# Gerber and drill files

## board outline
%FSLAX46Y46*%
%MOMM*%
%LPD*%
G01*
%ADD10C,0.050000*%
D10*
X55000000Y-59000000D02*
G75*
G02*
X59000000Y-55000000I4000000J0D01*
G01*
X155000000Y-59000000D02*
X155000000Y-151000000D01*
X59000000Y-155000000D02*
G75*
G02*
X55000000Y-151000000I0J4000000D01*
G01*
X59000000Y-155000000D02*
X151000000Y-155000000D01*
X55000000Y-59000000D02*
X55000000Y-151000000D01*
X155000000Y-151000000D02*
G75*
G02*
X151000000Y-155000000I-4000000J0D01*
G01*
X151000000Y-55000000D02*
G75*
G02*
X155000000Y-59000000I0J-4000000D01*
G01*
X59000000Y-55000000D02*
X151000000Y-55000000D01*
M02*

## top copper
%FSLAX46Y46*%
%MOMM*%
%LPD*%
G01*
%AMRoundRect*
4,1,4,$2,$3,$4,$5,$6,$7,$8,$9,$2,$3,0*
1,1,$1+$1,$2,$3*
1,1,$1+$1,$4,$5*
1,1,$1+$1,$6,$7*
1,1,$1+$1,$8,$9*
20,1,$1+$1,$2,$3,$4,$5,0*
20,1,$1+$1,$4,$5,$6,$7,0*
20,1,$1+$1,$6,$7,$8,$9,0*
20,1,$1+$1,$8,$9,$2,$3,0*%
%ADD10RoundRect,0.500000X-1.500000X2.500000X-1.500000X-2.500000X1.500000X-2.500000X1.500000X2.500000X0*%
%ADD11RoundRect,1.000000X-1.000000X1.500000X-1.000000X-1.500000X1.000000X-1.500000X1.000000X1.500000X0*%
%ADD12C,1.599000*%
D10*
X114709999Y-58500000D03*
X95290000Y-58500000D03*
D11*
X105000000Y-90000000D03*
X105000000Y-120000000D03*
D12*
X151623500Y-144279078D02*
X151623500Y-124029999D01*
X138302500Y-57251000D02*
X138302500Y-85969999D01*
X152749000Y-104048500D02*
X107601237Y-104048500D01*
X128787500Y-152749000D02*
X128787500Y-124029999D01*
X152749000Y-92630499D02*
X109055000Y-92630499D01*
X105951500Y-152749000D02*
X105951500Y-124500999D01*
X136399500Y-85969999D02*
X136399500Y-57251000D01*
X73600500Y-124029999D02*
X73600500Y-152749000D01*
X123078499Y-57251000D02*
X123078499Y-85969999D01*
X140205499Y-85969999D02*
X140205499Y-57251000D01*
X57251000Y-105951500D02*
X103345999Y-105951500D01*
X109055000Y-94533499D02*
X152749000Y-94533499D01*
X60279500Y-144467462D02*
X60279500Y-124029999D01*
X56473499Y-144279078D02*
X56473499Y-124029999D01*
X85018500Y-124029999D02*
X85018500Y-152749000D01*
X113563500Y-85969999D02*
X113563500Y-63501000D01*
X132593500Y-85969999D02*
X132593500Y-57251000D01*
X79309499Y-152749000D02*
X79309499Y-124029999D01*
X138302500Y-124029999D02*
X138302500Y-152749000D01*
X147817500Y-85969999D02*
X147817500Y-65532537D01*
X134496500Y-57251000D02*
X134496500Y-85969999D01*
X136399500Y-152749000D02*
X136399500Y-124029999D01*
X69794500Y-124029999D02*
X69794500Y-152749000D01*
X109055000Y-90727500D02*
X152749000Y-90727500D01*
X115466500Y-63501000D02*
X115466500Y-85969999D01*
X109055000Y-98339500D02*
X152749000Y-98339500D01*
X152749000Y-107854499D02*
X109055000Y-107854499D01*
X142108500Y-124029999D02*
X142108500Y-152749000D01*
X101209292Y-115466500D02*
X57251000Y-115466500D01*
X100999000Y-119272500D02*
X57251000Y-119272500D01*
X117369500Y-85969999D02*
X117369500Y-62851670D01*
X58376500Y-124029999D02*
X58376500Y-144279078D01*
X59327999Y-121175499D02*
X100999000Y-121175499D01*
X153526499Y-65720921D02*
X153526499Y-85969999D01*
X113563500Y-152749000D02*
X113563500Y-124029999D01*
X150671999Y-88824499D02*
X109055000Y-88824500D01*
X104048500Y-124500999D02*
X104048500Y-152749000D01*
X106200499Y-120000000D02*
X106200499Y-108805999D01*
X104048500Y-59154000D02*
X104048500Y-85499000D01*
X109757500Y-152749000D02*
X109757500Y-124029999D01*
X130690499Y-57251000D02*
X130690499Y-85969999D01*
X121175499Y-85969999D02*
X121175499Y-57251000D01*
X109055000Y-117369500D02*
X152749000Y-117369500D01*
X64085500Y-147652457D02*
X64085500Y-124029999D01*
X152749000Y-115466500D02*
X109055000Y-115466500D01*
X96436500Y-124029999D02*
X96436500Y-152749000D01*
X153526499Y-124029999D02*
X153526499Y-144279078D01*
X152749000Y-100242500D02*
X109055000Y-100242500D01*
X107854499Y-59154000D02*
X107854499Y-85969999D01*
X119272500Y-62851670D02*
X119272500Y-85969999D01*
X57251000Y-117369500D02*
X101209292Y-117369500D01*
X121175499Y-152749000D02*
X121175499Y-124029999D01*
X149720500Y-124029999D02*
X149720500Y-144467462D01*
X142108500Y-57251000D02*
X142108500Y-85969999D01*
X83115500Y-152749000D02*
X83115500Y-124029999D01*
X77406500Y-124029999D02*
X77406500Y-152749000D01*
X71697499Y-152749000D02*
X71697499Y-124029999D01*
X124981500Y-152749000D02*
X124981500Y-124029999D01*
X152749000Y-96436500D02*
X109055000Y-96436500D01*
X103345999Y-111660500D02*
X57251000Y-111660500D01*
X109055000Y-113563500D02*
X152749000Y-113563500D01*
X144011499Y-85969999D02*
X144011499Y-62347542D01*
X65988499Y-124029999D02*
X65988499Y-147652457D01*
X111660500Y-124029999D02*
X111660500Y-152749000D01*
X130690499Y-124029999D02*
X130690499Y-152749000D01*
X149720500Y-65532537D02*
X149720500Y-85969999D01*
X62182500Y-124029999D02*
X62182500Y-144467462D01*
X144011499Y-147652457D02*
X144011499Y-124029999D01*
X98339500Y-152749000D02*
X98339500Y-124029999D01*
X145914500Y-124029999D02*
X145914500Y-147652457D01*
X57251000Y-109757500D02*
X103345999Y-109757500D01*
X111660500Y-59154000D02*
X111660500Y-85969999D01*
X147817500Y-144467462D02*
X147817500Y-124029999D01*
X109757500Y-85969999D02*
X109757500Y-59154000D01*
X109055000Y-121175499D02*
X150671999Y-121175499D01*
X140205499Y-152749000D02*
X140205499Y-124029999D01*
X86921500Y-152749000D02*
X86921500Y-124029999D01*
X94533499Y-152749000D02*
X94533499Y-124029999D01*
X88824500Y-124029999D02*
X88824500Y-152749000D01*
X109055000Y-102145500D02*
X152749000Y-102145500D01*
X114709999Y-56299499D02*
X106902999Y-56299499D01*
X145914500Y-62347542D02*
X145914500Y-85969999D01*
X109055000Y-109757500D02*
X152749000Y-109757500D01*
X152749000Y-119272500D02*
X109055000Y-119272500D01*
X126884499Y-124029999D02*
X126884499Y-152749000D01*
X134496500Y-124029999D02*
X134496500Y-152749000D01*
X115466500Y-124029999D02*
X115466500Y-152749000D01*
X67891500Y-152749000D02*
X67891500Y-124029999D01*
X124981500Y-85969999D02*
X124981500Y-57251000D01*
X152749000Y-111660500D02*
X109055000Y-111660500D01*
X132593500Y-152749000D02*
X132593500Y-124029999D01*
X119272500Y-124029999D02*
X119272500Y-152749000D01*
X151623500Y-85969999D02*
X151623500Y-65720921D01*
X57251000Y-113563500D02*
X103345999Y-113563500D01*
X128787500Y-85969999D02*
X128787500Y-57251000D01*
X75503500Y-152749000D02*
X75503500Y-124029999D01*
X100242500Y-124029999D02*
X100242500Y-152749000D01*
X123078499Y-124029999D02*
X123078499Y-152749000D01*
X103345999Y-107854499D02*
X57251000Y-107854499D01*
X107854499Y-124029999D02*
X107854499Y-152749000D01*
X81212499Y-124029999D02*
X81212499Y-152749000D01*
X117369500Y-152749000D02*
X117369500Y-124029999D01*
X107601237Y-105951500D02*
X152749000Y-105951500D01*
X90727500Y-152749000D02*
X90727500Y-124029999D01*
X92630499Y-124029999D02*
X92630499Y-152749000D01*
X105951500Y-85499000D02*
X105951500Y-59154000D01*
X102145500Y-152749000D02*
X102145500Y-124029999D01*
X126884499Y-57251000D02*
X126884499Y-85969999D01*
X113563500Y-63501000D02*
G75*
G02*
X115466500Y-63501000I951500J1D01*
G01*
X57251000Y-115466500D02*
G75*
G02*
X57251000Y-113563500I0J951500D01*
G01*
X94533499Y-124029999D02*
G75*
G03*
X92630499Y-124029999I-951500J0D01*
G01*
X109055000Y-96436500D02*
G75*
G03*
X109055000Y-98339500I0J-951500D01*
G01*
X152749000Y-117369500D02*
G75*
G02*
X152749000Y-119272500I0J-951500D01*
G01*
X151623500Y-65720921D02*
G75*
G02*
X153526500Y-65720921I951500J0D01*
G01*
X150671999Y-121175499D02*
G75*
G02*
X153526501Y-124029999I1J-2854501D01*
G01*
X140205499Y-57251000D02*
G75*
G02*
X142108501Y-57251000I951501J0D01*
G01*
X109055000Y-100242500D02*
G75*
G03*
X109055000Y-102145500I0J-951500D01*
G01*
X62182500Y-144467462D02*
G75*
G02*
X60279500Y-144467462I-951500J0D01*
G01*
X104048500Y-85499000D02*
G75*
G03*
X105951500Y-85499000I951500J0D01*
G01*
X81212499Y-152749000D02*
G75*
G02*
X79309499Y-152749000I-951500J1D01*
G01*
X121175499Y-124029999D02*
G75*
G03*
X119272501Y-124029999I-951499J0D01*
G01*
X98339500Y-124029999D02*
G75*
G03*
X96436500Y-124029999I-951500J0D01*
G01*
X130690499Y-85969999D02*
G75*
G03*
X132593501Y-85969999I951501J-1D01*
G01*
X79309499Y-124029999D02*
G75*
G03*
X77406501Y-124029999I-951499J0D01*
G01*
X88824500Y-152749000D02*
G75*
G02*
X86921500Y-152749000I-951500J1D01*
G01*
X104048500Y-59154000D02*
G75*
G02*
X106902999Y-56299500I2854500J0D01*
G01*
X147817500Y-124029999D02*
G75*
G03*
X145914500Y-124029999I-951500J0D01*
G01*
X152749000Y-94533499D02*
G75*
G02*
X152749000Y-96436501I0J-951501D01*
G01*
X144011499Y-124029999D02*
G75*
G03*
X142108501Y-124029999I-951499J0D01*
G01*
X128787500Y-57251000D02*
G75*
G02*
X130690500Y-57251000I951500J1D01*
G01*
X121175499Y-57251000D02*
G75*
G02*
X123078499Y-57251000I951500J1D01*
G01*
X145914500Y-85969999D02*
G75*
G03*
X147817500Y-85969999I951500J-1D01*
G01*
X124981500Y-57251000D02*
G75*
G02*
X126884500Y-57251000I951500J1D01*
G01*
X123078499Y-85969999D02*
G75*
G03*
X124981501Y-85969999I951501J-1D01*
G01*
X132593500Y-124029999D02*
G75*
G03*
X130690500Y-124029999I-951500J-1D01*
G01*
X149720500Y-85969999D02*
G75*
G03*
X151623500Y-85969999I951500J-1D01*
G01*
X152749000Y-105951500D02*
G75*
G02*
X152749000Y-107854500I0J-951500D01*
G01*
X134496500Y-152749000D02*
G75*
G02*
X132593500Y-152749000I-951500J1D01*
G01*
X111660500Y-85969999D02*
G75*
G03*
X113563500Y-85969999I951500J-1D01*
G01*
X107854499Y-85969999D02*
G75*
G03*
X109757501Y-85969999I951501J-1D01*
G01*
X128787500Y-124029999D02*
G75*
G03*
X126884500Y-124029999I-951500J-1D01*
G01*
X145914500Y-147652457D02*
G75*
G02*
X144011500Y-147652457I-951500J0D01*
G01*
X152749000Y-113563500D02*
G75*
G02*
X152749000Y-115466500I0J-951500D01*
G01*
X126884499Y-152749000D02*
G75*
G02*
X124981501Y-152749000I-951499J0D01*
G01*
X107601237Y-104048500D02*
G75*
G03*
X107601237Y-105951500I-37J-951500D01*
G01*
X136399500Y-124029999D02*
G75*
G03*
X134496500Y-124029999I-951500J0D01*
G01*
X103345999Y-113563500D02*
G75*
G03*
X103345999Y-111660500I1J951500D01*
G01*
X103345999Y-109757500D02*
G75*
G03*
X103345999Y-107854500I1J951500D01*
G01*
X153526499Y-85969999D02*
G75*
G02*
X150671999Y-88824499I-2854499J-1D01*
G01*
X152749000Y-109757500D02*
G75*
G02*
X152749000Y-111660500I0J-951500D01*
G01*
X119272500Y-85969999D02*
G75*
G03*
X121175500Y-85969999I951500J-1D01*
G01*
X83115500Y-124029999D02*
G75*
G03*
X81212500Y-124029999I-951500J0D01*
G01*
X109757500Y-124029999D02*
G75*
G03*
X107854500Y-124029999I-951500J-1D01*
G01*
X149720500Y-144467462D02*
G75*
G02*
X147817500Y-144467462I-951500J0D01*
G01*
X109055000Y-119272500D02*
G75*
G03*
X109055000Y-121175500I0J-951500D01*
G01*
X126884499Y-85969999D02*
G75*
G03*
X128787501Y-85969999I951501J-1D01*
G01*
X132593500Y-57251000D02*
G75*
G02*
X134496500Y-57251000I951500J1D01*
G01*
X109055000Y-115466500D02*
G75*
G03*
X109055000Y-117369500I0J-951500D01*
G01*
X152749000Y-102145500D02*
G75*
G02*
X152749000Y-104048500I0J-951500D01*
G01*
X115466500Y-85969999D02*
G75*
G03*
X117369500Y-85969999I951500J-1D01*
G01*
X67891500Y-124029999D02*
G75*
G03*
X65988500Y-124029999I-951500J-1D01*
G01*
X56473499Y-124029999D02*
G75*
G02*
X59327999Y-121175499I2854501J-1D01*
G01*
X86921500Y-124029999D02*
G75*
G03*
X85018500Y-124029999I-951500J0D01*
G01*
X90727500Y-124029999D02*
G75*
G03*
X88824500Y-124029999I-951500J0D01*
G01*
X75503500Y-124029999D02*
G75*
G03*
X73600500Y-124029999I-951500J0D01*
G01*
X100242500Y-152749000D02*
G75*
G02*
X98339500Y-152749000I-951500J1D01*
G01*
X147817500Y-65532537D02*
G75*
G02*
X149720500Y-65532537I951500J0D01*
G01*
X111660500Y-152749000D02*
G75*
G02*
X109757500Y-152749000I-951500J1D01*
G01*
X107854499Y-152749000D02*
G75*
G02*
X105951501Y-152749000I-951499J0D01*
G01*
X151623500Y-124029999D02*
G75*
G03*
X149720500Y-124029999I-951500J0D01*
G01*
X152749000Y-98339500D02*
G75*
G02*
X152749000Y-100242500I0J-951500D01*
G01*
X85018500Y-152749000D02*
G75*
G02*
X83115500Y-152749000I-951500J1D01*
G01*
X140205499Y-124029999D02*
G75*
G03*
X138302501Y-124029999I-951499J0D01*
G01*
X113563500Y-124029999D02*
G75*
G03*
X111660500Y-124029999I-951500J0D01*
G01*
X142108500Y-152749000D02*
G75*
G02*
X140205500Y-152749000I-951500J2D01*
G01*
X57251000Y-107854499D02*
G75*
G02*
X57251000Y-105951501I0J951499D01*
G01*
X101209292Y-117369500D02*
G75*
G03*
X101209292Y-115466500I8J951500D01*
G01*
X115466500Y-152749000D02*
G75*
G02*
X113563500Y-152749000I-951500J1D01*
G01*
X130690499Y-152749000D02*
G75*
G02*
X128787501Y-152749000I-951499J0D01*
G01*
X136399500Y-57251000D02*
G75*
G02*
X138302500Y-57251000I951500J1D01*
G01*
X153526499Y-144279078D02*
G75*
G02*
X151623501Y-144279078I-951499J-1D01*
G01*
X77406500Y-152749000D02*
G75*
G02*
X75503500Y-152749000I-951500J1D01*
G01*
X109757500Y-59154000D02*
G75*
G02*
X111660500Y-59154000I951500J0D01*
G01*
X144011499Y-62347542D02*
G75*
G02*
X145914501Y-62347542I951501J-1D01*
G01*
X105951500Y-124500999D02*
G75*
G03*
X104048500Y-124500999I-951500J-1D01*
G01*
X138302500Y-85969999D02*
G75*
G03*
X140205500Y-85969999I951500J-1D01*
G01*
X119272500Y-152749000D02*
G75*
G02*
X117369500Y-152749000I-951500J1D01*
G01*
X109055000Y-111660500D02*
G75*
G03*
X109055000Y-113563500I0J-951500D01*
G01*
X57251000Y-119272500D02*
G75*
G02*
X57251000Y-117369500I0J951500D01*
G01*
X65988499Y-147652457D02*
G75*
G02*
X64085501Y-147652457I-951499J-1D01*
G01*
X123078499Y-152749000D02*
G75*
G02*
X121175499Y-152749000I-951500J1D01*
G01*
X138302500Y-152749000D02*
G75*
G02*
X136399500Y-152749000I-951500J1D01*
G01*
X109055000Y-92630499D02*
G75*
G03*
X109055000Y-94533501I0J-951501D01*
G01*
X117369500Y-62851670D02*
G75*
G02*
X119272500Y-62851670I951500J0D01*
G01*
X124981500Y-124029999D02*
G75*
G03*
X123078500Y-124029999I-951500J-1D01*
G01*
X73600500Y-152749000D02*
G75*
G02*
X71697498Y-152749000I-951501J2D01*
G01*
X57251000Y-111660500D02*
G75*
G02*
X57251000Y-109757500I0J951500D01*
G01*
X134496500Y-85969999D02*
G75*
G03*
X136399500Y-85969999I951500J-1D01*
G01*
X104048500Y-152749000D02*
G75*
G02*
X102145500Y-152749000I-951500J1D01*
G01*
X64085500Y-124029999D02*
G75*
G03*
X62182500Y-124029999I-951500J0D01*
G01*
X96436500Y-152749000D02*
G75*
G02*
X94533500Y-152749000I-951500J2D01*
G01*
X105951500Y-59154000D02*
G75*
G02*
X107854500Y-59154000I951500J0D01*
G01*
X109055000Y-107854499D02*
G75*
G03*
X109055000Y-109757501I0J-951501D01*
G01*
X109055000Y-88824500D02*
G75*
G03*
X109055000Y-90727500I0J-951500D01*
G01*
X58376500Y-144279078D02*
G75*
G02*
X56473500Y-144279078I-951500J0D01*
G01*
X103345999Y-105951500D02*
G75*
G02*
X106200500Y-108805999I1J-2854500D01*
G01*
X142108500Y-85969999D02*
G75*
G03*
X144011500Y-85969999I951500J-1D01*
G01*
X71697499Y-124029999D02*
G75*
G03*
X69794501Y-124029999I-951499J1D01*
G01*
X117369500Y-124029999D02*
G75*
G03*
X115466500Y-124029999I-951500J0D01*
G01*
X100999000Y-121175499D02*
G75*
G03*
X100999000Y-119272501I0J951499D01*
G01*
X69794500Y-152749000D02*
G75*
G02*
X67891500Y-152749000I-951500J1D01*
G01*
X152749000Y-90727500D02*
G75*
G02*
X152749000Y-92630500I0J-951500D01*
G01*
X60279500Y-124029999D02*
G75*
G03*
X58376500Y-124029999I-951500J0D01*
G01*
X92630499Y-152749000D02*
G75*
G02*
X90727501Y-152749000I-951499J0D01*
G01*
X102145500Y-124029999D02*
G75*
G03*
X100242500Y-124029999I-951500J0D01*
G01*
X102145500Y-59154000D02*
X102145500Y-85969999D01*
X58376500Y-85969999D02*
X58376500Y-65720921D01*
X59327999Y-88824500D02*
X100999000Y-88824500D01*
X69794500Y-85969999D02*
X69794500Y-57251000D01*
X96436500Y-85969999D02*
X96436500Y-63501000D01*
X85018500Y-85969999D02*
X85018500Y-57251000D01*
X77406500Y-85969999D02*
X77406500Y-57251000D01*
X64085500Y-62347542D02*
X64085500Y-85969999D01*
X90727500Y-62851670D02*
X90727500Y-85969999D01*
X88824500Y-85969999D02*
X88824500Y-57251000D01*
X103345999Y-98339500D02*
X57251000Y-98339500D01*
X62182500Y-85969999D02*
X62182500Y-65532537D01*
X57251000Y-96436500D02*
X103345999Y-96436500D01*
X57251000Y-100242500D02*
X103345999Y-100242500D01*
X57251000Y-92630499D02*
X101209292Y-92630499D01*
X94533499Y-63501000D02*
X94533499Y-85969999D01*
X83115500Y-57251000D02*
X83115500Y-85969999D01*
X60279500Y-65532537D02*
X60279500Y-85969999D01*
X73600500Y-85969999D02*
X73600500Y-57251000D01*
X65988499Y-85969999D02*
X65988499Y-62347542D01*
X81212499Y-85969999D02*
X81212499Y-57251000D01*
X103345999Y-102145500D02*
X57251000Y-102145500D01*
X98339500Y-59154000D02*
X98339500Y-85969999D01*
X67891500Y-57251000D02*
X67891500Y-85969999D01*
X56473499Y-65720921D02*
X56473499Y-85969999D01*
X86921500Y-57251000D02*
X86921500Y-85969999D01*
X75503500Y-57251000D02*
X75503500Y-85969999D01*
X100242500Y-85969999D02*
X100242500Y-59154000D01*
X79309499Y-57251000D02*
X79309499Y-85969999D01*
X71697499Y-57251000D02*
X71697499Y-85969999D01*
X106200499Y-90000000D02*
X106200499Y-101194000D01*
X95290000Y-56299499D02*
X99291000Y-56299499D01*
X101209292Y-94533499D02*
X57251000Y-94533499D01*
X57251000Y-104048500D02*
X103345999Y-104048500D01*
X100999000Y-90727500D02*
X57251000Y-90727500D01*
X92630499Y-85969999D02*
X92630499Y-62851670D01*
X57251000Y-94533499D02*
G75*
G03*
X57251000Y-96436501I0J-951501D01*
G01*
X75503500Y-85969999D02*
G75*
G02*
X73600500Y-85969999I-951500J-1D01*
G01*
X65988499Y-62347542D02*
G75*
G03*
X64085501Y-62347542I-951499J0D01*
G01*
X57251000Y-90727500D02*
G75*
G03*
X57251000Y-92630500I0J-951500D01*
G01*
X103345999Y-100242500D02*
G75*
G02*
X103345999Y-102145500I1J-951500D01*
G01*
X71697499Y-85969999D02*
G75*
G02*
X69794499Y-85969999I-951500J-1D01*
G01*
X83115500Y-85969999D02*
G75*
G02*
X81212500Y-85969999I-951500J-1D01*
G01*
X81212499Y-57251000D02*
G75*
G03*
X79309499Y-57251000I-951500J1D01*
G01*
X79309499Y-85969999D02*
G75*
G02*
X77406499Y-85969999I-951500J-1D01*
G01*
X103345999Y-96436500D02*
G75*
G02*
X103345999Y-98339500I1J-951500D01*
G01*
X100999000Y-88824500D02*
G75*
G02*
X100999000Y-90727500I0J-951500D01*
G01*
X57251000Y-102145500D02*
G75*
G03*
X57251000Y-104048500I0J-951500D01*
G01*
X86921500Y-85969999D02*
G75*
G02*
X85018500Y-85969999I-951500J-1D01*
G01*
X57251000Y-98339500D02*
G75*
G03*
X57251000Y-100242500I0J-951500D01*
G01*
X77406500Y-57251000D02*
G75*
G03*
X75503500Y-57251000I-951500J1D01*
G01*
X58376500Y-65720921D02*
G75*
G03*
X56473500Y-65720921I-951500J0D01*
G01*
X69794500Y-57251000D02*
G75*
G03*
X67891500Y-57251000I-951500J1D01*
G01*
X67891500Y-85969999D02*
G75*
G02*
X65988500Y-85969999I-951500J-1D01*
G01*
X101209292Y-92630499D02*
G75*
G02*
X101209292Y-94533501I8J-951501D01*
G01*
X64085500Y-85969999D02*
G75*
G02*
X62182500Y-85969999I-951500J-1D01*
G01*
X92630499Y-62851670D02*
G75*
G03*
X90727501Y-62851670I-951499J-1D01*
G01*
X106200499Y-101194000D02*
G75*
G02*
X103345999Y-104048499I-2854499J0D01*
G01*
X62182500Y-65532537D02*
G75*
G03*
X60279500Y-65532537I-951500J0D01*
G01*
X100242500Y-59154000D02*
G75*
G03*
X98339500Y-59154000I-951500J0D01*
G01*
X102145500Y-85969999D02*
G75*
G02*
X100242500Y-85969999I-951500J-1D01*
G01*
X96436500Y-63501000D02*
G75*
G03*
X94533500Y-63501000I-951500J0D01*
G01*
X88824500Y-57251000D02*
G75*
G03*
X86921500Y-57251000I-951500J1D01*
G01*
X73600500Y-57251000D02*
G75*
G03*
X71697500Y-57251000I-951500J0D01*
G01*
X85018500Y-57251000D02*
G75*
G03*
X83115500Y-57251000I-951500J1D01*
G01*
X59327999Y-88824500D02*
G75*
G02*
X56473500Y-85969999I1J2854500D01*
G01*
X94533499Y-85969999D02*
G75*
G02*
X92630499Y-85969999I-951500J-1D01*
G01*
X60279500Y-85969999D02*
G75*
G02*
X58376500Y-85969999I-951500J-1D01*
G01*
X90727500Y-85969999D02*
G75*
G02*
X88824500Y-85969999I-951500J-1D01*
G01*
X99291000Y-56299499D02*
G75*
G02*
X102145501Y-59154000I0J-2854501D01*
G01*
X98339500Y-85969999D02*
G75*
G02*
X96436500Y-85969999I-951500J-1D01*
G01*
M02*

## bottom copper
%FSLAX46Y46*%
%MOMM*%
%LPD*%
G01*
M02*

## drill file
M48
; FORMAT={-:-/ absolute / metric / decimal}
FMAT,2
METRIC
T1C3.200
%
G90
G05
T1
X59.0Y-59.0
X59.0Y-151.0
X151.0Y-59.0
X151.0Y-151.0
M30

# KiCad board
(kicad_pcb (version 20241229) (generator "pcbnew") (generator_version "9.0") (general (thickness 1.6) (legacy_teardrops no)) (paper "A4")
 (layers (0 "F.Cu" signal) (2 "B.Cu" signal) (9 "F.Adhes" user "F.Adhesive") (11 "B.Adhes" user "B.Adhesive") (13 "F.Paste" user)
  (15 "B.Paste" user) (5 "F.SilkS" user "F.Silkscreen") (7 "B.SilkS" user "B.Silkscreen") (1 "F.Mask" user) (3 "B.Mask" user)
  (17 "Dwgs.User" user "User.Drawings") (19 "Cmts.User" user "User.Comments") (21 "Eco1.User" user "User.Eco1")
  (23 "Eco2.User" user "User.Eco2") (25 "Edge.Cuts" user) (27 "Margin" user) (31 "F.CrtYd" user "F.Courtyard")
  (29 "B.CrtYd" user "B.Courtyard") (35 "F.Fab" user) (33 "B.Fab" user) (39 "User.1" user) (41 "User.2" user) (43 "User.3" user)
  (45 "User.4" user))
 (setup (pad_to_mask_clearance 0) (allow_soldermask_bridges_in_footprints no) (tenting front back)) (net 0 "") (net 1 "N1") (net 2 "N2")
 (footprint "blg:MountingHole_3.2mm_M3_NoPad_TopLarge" (layer "F.Cu") (at 151 59)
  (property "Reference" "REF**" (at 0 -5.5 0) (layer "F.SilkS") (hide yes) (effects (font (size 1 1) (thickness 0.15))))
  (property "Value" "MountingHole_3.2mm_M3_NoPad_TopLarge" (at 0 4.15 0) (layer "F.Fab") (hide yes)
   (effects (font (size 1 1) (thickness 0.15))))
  (pad "" np_thru_hole circle (at 0 0) (size 7.6 7.6) (drill 3.2) (layers) (zone_connect 2)))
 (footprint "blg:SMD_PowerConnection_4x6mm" (layer "F.Cu") (at 114.709999 58.5 -90)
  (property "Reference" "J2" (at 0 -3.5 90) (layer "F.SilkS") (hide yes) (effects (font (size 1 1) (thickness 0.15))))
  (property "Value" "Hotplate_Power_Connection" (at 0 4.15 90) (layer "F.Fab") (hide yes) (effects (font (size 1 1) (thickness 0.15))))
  (pad "1" smd roundrect (at 0 0 270) (size 6 4) (layers "F.Cu" "F.Mask" "F.Paste") (roundrect_rratio 0.125) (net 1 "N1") (zone_connect 2)))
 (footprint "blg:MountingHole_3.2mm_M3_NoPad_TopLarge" (layer "F.Cu") (at 59 151)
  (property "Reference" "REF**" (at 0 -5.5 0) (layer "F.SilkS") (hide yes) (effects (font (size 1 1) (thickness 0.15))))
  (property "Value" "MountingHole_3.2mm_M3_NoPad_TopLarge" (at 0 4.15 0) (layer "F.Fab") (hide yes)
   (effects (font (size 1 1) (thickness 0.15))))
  (pad "" np_thru_hole circle (at 0 0) (size 7.6 7.6) (drill 3.2) (layers) (zone_connect 2)))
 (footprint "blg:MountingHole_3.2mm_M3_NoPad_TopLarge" (layer "F.Cu") (at 151 151)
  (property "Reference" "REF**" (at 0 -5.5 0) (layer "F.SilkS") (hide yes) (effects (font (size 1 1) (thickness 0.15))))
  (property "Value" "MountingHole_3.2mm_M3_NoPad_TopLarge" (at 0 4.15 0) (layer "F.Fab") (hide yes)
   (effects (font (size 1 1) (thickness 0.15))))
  (pad "" np_thru_hole circle (at 0 0) (size 7.6 7.6) (drill 3.2) (layers) (zone_connect 2)))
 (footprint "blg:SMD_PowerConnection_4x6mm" (layer "F.Cu") (at 95.29 58.5 -90)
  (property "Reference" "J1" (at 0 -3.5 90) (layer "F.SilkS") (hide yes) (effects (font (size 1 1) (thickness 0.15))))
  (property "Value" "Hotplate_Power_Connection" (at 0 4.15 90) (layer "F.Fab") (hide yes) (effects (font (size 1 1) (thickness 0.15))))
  (pad "1" smd roundrect (at 0 0 270) (size 6 4) (layers "F.Cu" "F.Mask" "F.Paste") (roundrect_rratio 0.125) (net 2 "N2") (zone_connect 2)))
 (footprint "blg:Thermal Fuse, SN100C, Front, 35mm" (layer "F.Cu") (at 105 105 -90)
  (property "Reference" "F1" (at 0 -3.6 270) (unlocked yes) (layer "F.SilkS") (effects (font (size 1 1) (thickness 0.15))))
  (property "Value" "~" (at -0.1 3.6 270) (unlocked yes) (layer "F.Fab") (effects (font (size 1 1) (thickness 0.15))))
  (pad "1" smd roundrect (at -15 0 270) (size 5 4) (layers "F.Cu" "F.Mask") (roundrect_rratio 0.25) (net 2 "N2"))
  (pad "2" smd roundrect (at 15 0 270) (size 5 4) (layers "F.Cu" "F.Mask") (roundrect_rratio 0.25) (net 1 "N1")))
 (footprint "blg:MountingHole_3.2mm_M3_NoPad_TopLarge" (layer "F.Cu") (at 59 59)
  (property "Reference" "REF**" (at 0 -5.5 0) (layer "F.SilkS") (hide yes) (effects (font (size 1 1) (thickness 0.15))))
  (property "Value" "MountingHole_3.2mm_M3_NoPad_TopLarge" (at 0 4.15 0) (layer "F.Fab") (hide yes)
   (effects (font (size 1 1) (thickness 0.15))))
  (pad "" np_thru_hole circle (at 0 0) (size 7.6 7.6) (drill 3.2) (layers) (zone_connect 2)))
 (gr_arc (start 55 59) (mid 56.171573 56.171573) (end 59 55) (stroke (width 0.05) (type solid)) (layer "Edge.Cuts"))
 (gr_line (start 155 59) (end 155 151) (stroke (width 0.05) (type default)) (layer "Edge.Cuts"))
 (gr_arc (start 59 155) (mid 56.171573 153.828427) (end 55 151) (stroke (width 0.05) (type solid)) (layer "Edge.Cuts"))
 (gr_line (start 59 155) (end 151 155) (stroke (width 0.05) (type default)) (layer "Edge.Cuts"))
 (gr_line (start 55 59) (end 55 151) (stroke (width 0.05) (type default)) (layer "Edge.Cuts"))
 (gr_arc (start 155 151) (mid 153.828427 153.828427) (end 151 155) (stroke (width 0.05) (type solid)) (layer "Edge.Cuts"))
 (gr_arc (start 151 55) (mid 153.828427 56.171573) (end 155 59) (stroke (width 0.05) (type solid)) (layer "Edge.Cuts"))
 (gr_line (start 59 55) (end 151 55) (stroke (width 0.05) (type default)) (layer "Edge.Cuts"))
 (segment (start 151.6235 144.279078) (end 151.6235 124.029999) (width 1.599) (layer "F.Cu") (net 1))
 (segment (start 138.3025 57.251) (end 138.3025 85.969999) (width 1.599) (layer "F.Cu") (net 1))
 (segment (start 152.749 104.0485) (end 107.601237 104.0485) (width 1.599) (layer "F.Cu") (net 1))
 (segment (start 128.7875 152.749) (end 128.7875 124.029999) (width 1.599) (layer "F.Cu") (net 1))
 (segment (start 152.749 92.630499) (end 109.055 92.630499) (width 1.599) (layer "F.Cu") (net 1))
 (segment (start 105.9515 152.749) (end 105.9515 124.500999) (width 1.599) (layer "F.Cu") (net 1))
 (segment (start 136.3995 85.969999) (end 136.3995 57.251) (width 1.599) (layer "F.Cu") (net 1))
 (segment (start 73.6005 124.029999) (end 73.6005 152.749) (width 1.599) (layer "F.Cu") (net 1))
 (segment (start 123.078499 57.251) (end 123.078499 85.969999) (width 1.599) (layer "F.Cu") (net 1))
 (segment (start 140.205499 85.969999) (end 140.205499 57.251) (width 1.599) (layer "F.Cu") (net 1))
 (segment (start 57.251 105.9515) (end 103.345999 105.9515) (width 1.599) (layer "F.Cu") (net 1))
 (segment (start 109.055 94.533499) (end 152.749 94.533499) (width 1.599) (layer "F.Cu") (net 1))
 (segment (start 60.2795 144.467462) (end 60.2795 124.029999) (width 1.599) (layer "F.Cu") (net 1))
 (segment (start 56.473499 144.279078) (end 56.473499 124.029999) (width 1.599) (layer "F.Cu") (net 1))
 (segment (start 85.0185 124.029999) (end 85.0185 152.749) (width 1.599) (layer "F.Cu") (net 1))
 (segment (start 113.5635 85.969999) (end 113.5635 63.501) (width 1.599) (layer "F.Cu") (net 1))
 (segment (start 132.5935 85.969999) (end 132.5935 57.251) (width 1.599) (layer "F.Cu") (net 1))
 (segment (start 79.309499 152.749) (end 79.309499 124.029999) (width 1.599) (layer "F.Cu") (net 1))
 (segment (start 138.3025 124.029999) (end 138.3025 152.749) (width 1.599) (layer "F.Cu") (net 1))
 (segment (start 147.8175 85.969999) (end 147.8175 65.532537) (width 1.599) (layer "F.Cu") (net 1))
 (segment (start 134.4965 57.251) (end 134.4965 85.969999) (width 1.599) (layer "F.Cu") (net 1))
 (segment (start 136.3995 152.749) (end 136.3995 124.029999) (width 1.599) (layer "F.Cu") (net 1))
 (segment (start 69.7945 124.029999) (end 69.7945 152.749) (width 1.599) (layer "F.Cu") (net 1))
 (segment (start 109.055 90.7275) (end 152.749 90.7275) (width 1.599) (layer "F.Cu") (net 1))
 (segment (start 115.4665 63.501) (end 115.4665 85.969999) (width 1.599) (layer "F.Cu") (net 1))
 (segment (start 109.055 98.3395) (end 152.749 98.3395) (width 1.599) (layer "F.Cu") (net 1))
 (segment (start 152.749 107.854499) (end 109.055 107.854499) (width 1.599) (layer "F.Cu") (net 1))
 (segment (start 142.1085 124.029999) (end 142.1085 152.749) (width 1.599) (layer "F.Cu") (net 1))
 (segment (start 101.209292 115.4665) (end 57.251 115.4665) (width 1.599) (layer "F.Cu") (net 1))
 (segment (start 100.999 119.2725) (end 57.251 119.2725) (width 1.599) (layer "F.Cu") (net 1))
 (segment (start 117.3695 85.969999) (end 117.3695 62.85167) (width 1.599) (layer "F.Cu") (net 1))
 (segment (start 58.3765 124.029999) (end 58.3765 144.279078) (width 1.599) (layer "F.Cu") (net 1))
 (segment (start 59.327999 121.175499) (end 100.999 121.175499) (width 1.599) (layer "F.Cu") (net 1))
 (segment (start 153.526499 65.720921) (end 153.526499 85.969999) (width 1.599) (layer "F.Cu") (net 1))
 (segment (start 113.5635 152.749) (end 113.5635 124.029999) (width 1.599) (layer "F.Cu") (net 1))
 (segment (start 150.671999 88.824499) (end 109.055 88.8245) (width 1.599) (layer "F.Cu") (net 1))
 (segment (start 104.0485 124.500999) (end 104.0485 152.749) (width 1.599) (layer "F.Cu") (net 1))
 (segment (start 106.200499 120) (end 106.200499 108.805999) (width 1.599) (layer "F.Cu") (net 1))
 (segment (start 104.0485 59.154) (end 104.0485 85.499) (width 1.599) (layer "F.Cu") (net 1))
 (segment (start 109.7575 152.749) (end 109.7575 124.029999) (width 1.599) (layer "F.Cu") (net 1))
 (segment (start 130.690499 57.251) (end 130.690499 85.969999) (width 1.599) (layer "F.Cu") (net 1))
 (segment (start 121.175499 85.969999) (end 121.175499 57.251) (width 1.599) (layer "F.Cu") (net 1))
 (segment (start 109.055 117.3695) (end 152.749 117.3695) (width 1.599) (layer "F.Cu") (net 1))
 (segment (start 64.0855 147.652457) (end 64.0855 124.029999) (width 1.599) (layer "F.Cu") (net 1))
 (segment (start 152.749 115.4665) (end 109.055 115.4665) (width 1.599) (layer "F.Cu") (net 1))
 (segment (start 96.4365 124.029999) (end 96.4365 152.749) (width 1.599) (layer "F.Cu") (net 1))
 (segment (start 153.526499 124.029999) (end 153.526499 144.279078) (width 1.599) (layer "F.Cu") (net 1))
 (segment (start 152.749 100.2425) (end 109.055 100.2425) (width 1.599) (layer "F.Cu") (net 1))
 (segment (start 107.854499 59.154) (end 107.854499 85.969999) (width 1.599) (layer "F.Cu") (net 1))
 (segment (start 119.2725 62.85167) (end 119.2725 85.969999) (width 1.599) (layer "F.Cu") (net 1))
 (segment (start 57.251 117.3695) (end 101.209292 117.3695) (width 1.599) (layer "F.Cu") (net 1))
 (segment (start 121.175499 152.749) (end 121.175499 124.029999) (width 1.599) (layer "F.Cu") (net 1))
 (segment (start 149.7205 124.029999) (end 149.7205 144.467462) (width 1.599) (layer "F.Cu") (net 1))
 (segment (start 142.1085 57.251) (end 142.1085 85.969999) (width 1.599) (layer "F.Cu") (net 1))
 (segment (start 83.1155 152.749) (end 83.1155 124.029999) (width 1.599) (layer "F.Cu") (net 1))
 (segment (start 77.4065 124.029999) (end 77.4065 152.749) (width 1.599) (layer "F.Cu") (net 1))
 (segment (start 71.697499 152.749) (end 71.697499 124.029999) (width 1.599) (layer "F.Cu") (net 1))
 (segment (start 124.9815 152.749) (end 124.9815 124.029999) (width 1.599) (layer "F.Cu") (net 1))
 (segment (start 152.749 96.4365) (end 109.055 96.4365) (width 1.599) (layer "F.Cu") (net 1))
 (segment (start 103.345999 111.6605) (end 57.251 111.6605) (width 1.599) (layer "F.Cu") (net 1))
 (segment (start 109.055 113.5635) (end 152.749 113.5635) (width 1.599) (layer "F.Cu") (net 1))
 (segment (start 144.011499 85.969999) (end 144.011499 62.347542) (width 1.599) (layer "F.Cu") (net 1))
 (segment (start 65.988499 124.029999) (end 65.988499 147.652457) (width 1.599) (layer "F.Cu") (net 1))
 (segment (start 111.6605 124.029999) (end 111.6605 152.749) (width 1.599) (layer "F.Cu") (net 1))
 (segment (start 130.690499 124.029999) (end 130.690499 152.749) (width 1.599) (layer "F.Cu") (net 1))
 (segment (start 149.7205 65.532537) (end 149.7205 85.969999) (width 1.599) (layer "F.Cu") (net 1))
 (segment (start 62.1825 124.029999) (end 62.1825 144.467462) (width 1.599) (layer "F.Cu") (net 1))
 (segment (start 144.011499 147.652457) (end 144.011499 124.029999) (width 1.599) (layer "F.Cu") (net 1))
 (segment (start 98.3395 152.749) (end 98.3395 124.029999) (width 1.599) (layer "F.Cu") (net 1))
 (segment (start 145.9145 124.029999) (end 145.9145 147.652457) (width 1.599) (layer "F.Cu") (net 1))
 (segment (start 57.251 109.7575) (end 103.345999 109.7575) (width 1.599) (layer "F.Cu") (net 1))
 (segment (start 111.6605 59.154) (end 111.6605 85.969999) (width 1.599) (layer "F.Cu") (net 1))
 (segment (start 147.8175 144.467462) (end 147.8175 124.029999) (width 1.599) (layer "F.Cu") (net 1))
 (segment (start 109.7575 85.969999) (end 109.7575 59.154) (width 1.599) (layer "F.Cu") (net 1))
 (segment (start 109.055 121.175499) (end 150.671999 121.175499) (width 1.599) (layer "F.Cu") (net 1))
 (segment (start 140.205499 152.749) (end 140.205499 124.029999) (width 1.599) (layer "F.Cu") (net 1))
 (segment (start 86.9215 152.749) (end 86.9215 124.029999) (width 1.599) (layer "F.Cu") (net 1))
 (segment (start 94.533499 152.749) (end 94.533499 124.029999) (width 1.599) (layer "F.Cu") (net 1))
 (segment (start 88.8245 124.029999) (end 88.8245 152.749) (width 1.599) (layer "F.Cu") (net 1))
 (segment (start 109.055 102.1455) (end 152.749 102.1455) (width 1.599) (layer "F.Cu") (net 1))
 (segment (start 114.709999 56.299499) (end 106.902999 56.299499) (width 1.599) (layer "F.Cu") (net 1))
 (segment (start 145.9145 62.347542) (end 145.9145 85.969999) (width 1.599) (layer "F.Cu") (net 1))
 (segment (start 109.055 109.7575) (end 152.749 109.7575) (width 1.599) (layer "F.Cu") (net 1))
 (segment (start 152.749 119.2725) (end 109.055 119.2725) (width 1.599) (layer "F.Cu") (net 1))
 (segment (start 126.884499 124.029999) (end 126.884499 152.749) (width 1.599) (layer "F.Cu") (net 1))
 (segment (start 134.4965 124.029999) (end 134.4965 152.749) (width 1.599) (layer "F.Cu") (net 1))
 (segment (start 115.4665 124.029999) (end 115.4665 152.749) (width 1.599) (layer "F.Cu") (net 1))
 (segment (start 67.8915 152.749) (end 67.8915 124.029999) (width 1.599) (layer "F.Cu") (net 1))
 (segment (start 124.9815 85.969999) (end 124.9815 57.251) (width 1.599) (layer "F.Cu") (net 1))
 (segment (start 152.749 111.6605) (end 109.055 111.6605) (width 1.599) (layer "F.Cu") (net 1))
 (segment (start 132.5935 152.749) (end 132.5935 124.029999) (width 1.599) (layer "F.Cu") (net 1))
 (segment (start 119.2725 124.029999) (end 119.2725 152.749) (width 1.599) (layer "F.Cu") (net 1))
 (segment (start 151.6235 85.969999) (end 151.6235 65.720921) (width 1.599) (layer "F.Cu") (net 1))
 (segment (start 57.251 113.5635) (end 103.345999 113.5635) (width 1.599) (layer "F.Cu") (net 1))
 (segment (start 128.7875 85.969999) (end 128.7875 57.251) (width 1.599) (layer "F.Cu") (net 1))
 (segment (start 75.5035 152.749) (end 75.5035 124.029999) (width 1.599) (layer "F.Cu") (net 1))
 (segment (start 100.2425 124.029999) (end 100.2425 152.749) (width 1.599) (layer "F.Cu") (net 1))
 (segment (start 123.078499 124.029999) (end 123.078499 152.749) (width 1.599) (layer "F.Cu") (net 1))
 (segment (start 103.345999 107.854499) (end 57.251 107.854499) (width 1.599) (layer "F.Cu") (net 1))
 (segment (start 107.854499 124.029999) (end 107.854499 152.749) (width 1.599) (layer "F.Cu") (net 1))
 (segment (start 81.212499 124.029999) (end 81.212499 152.749) (width 1.599) (layer "F.Cu") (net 1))
 (segment (start 117.3695 152.749) (end 117.3695 124.029999) (width 1.599) (layer "F.Cu") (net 1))
 (segment (start 107.601237 105.9515) (end 152.749 105.9515) (width 1.599) (layer "F.Cu") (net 1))
 (segment (start 90.7275 152.749) (end 90.7275 124.029999) (width 1.599) (layer "F.Cu") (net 1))
 (segment (start 92.630499 124.029999) (end 92.630499 152.749) (width 1.599) (layer "F.Cu") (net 1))
 (segment (start 105.9515 85.499) (end 105.9515 59.154) (width 1.599) (layer "F.Cu") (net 1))
 (segment (start 102.1455 152.749) (end 102.1455 124.029999) (width 1.599) (layer "F.Cu") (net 1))
 (segment (start 126.884499 57.251) (end 126.884499 85.969999) (width 1.599) (layer "F.Cu") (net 1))
 (arc (start 113.5635 63.501) (mid 114.514999 62.549499) (end 115.4665 63.501) (width 1.599) (layer "F.Cu") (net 1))
 (arc (start 57.251 115.4665) (mid 56.299499 114.514999) (end 57.251 113.5635) (width 1.599) (layer "F.Cu") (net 1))
 (arc (start 94.533499 124.029999) (mid 93.582 123.078499) (end 92.630499 124.029999) (width 1.599) (layer "F.Cu") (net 1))
 (arc (start 109.055 96.4365) (mid 108.1035 97.388) (end 109.055 98.3395) (width 1.599) (layer "F.Cu") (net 1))
 (arc (start 152.749 117.3695) (mid 153.700499 118.321) (end 152.749 119.2725) (width 1.599) (layer "F.Cu") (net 1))
 (arc (start 151.6235 65.720921) (mid 152.575 64.769421) (end 153.526499 65.720921) (width 1.599) (layer "F.Cu") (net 1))
 (arc (start 150.671999 121.175499) (mid 152.690436 122.011563) (end 153.526499 124.029999) (width 1.599) (layer "F.Cu") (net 1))
 (arc (start 140.205499 57.251) (mid 141.157 56.299499) (end 142.1085 57.251) (width 1.599) (layer "F.Cu") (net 1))
 (arc (start 109.055 100.2425) (mid 108.1035 101.193999) (end 109.055 102.1455) (width 1.599) (layer "F.Cu") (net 1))
 (arc (start 62.1825 144.467462) (mid 61.230999 145.418962) (end 60.2795 144.467462) (width 1.599) (layer "F.Cu") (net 1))
 (arc (start 104.0485 85.499) (mid 105 86.4505) (end 105.9515 85.499) (width 1.599) (layer "F.Cu") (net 1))
 (arc (start 81.212499 152.749) (mid 80.261 153.700499) (end 79.309499 152.749) (width 1.599) (layer "F.Cu") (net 1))
 (arc (start 121.175499 124.029999) (mid 120.224 123.078499) (end 119.2725 124.029999) (width 1.599) (layer "F.Cu") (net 1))
 (arc (start 98.3395 124.029999) (mid 97.388 123.078499) (end 96.4365 124.029999) (width 1.599) (layer "F.Cu") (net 1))
 (arc (start 130.690499 85.969999) (mid 131.641999 86.9215) (end 132.5935 85.969999) (width 1.599) (layer "F.Cu") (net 1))
 (arc (start 79.309499 124.029999) (mid 78.358 123.078499) (end 77.4065 124.029999) (width 1.599) (layer "F.Cu") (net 1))
 (arc (start 88.8245 152.749) (mid 87.872999 153.700499) (end 86.9215 152.749) (width 1.599) (layer "F.Cu") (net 1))
 (arc (start 104.0485 59.154) (mid 104.884563 57.135563) (end 106.902999 56.299499) (width 1.599) (layer "F.Cu") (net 1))
 (arc (start 147.8175 124.029999) (mid 146.866 123.078499) (end 145.9145 124.029999) (width 1.599) (layer "F.Cu") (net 1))
 (arc (start 152.749 94.533499) (mid 153.700499 95.485) (end 152.749 96.4365) (width 1.599) (layer "F.Cu") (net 1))
 (arc (start 144.011499 124.029999) (mid 143.06 123.078499) (end 142.1085 124.029999) (width 1.599) (layer "F.Cu") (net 1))
 (arc (start 128.7875 57.251) (mid 129.739 56.299499) (end 130.690499 57.251) (width 1.599) (layer "F.Cu") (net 1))
 (arc (start 121.175499 57.251) (mid 122.127 56.299499) (end 123.078499 57.251) (width 1.599) (layer "F.Cu") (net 1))
 (arc (start 145.9145 85.969999) (mid 146.866 86.9215) (end 147.8175 85.969999) (width 1.599) (layer "F.Cu") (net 1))
 (arc (start 124.9815 57.251) (mid 125.933 56.299499) (end 126.884499 57.251) (width 1.599) (layer "F.Cu") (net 1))
 (arc (start 123.078499 85.969999) (mid 124.029999 86.9215) (end 124.9815 85.969999) (width 1.599) (layer "F.Cu") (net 1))
 (arc (start 132.5935 124.029999) (mid 131.641999 123.078499) (end 130.690499 124.029999) (width 1.599) (layer "F.Cu") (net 1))
 (arc (start 149.7205 85.969999) (mid 150.672 86.9215) (end 151.6235 85.969999) (width 1.599) (layer "F.Cu") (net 1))
 (arc (start 152.749 105.9515) (mid 153.700499 106.902999) (end 152.749 107.854499) (width 1.599) (layer "F.Cu") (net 1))
 (arc (start 134.4965 152.749) (mid 133.544999 153.700499) (end 132.5935 152.749) (width 1.599) (layer "F.Cu") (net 1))
 (arc (start 111.6605 85.969999) (mid 112.612 86.9215) (end 113.5635 85.969999) (width 1.599) (layer "F.Cu") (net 1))
 (arc (start 107.854499 85.969999) (mid 108.806 86.9215) (end 109.7575 85.969999) (width 1.599) (layer "F.Cu") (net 1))
 (arc (start 128.7875 124.029999) (mid 127.836 123.078499) (end 126.884499 124.029999) (width 1.599) (layer "F.Cu") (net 1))
 (arc (start 145.9145 147.652457) (mid 144.963 148.603957) (end 144.011499 147.652457) (width 1.599) (layer "F.Cu") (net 1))
 (arc (start 152.749 113.5635) (mid 153.700499 114.514999) (end 152.749 115.4665) (width 1.599) (layer "F.Cu") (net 1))
 (arc (start 126.884499 152.749) (mid 125.933 153.700499) (end 124.9815 152.749) (width 1.599) (layer "F.Cu") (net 1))
 (arc (start 107.601237 104.0485) (mid 106.649736 105) (end 107.601237 105.9515) (width 1.599) (layer "F.Cu") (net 1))
 (arc (start 136.3995 124.029999) (mid 135.447999 123.078499) (end 134.4965 124.029999) (width 1.599) (layer "F.Cu") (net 1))
 (arc (start 103.345999 113.5635) (mid 104.2975 112.612) (end 103.345999 111.6605) (width 1.599) (layer "F.Cu") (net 1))
 (arc (start 103.345999 109.7575) (mid 104.2975 108.806) (end 103.345999 107.854499) (width 1.599) (layer "F.Cu") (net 1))
 (arc (start 153.526499 85.969999) (mid 152.690436 87.988436) (end 150.671999 88.824499) (width 1.599) (layer "F.Cu") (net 1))
 (arc (start 152.749 109.7575) (mid 153.700499 110.709) (end 152.749 111.6605) (width 1.599) (layer "F.Cu") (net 1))
 (arc (start 119.2725 85.969999) (mid 120.224 86.9215) (end 121.175499 85.969999) (width 1.599) (layer "F.Cu") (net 1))
 (arc (start 83.1155 124.029999) (mid 82.164 123.078499) (end 81.212499 124.029999) (width 1.599) (layer "F.Cu") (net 1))
 (arc (start 109.7575 124.029999) (mid 108.806 123.078499) (end 107.854499 124.029999) (width 1.599) (layer "F.Cu") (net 1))
 (arc (start 149.7205 144.467462) (mid 148.768999 145.418962) (end 147.8175 144.467462) (width 1.599) (layer "F.Cu") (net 1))
 (arc (start 109.055 119.2725) (mid 108.1035 120.224) (end 109.055 121.175499) (width 1.599) (layer "F.Cu") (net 1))
 (arc (start 126.884499 85.969999) (mid 127.836 86.9215) (end 128.7875 85.969999) (width 1.599) (layer "F.Cu") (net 1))
 (arc (start 132.5935 57.251) (mid 133.544999 56.299499) (end 134.4965 57.251) (width 1.599) (layer "F.Cu") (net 1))
 (arc (start 109.055 115.4665) (mid 108.1035 116.417999) (end 109.055 117.3695) (width 1.599) (layer "F.Cu") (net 1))
 (arc (start 152.749 102.1455) (mid 153.700499 103.097) (end 152.749 104.0485) (width 1.599) (layer "F.Cu") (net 1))
 (arc (start 115.4665 85.969999) (mid 116.417999 86.9215) (end 117.3695 85.969999) (width 1.599) (layer "F.Cu") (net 1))
 (arc (start 67.8915 124.029999) (mid 66.94 123.078499) (end 65.988499 124.029999) (width 1.599) (layer "F.Cu") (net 1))
 (arc (start 56.473499 124.029999) (mid 57.309563 122.011563) (end 59.327999 121.175499) (width 1.599) (layer "F.Cu") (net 1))
 (arc (start 86.9215 124.029999) (mid 85.969999 123.078499) (end 85.0185 124.029999) (width 1.599) (layer "F.Cu") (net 1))
 (arc (start 90.7275 124.029999) (mid 89.776 123.078499) (end 88.8245 124.029999) (width 1.599) (layer "F.Cu") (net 1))
 (arc (start 75.5035 124.029999) (mid 74.551999 123.078499) (end 73.6005 124.029999) (width 1.599) (layer "F.Cu") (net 1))
 (arc (start 100.2425 152.749) (mid 99.291 153.700499) (end 98.3395 152.749) (width 1.599) (layer "F.Cu") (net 1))
 (arc (start 147.8175 65.532537) (mid 148.768999 64.581037) (end 149.7205 65.532537) (width 1.599) (layer "F.Cu") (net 1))
 (arc (start 111.6605 152.749) (mid 110.709 153.700499) (end 109.7575 152.749) (width 1.599) (layer "F.Cu") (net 1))
 (arc (start 107.854499 152.749) (mid 106.902999 153.700499) (end 105.9515 152.749) (width 1.599) (layer "F.Cu") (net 1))
 (arc (start 151.6235 124.029999) (mid 150.672 123.078499) (end 149.7205 124.029999) (width 1.599) (layer "F.Cu") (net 1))
 (arc (start 152.749 98.3395) (mid 153.700499 99.291) (end 152.749 100.2425) (width 1.599) (layer "F.Cu") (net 1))
 (arc (start 85.0185 152.749) (mid 84.067 153.700499) (end 83.1155 152.749) (width 1.599) (layer "F.Cu") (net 1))
 (arc (start 140.205499 124.029999) (mid 139.254 123.078499) (end 138.3025 124.029999) (width 1.599) (layer "F.Cu") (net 1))
 (arc (start 113.5635 124.029999) (mid 112.612 123.078499) (end 111.6605 124.029999) (width 1.599) (layer "F.Cu") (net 1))
 (arc (start 142.1085 152.749) (mid 141.157 153.700499) (end 140.205499 152.749) (width 1.599) (layer "F.Cu") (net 1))
 (arc (start 57.251 107.854499) (mid 56.299499 106.902999) (end 57.251 105.9515) (width 1.599) (layer "F.Cu") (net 1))
 (arc (start 101.209292 117.3695) (mid 102.160793 116.417999) (end 101.209292 115.4665) (width 1.599) (layer "F.Cu") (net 1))
 (arc (start 115.4665 152.749) (mid 114.514999 153.700499) (end 113.5635 152.749) (width 1.599) (layer "F.Cu") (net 1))
 (arc (start 130.690499 152.749) (mid 129.739 153.700499) (end 128.7875 152.749) (width 1.599) (layer "F.Cu") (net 1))
 (arc (start 136.3995 57.251) (mid 137.351 56.299499) (end 138.3025 57.251) (width 1.599) (layer "F.Cu") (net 1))
 (arc (start 153.526499 144.279078) (mid 152.575 145.230578) (end 151.6235 144.279078) (width 1.599) (layer "F.Cu") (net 1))
 (arc (start 77.4065 152.749) (mid 76.455 153.700499) (end 75.5035 152.749) (width 1.599) (layer "F.Cu") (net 1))
 (arc (start 109.7575 59.154) (mid 110.709 58.2025) (end 111.6605 59.154) (width 1.599) (layer "F.Cu") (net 1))
 (arc (start 144.011499 62.347542) (mid 144.963 61.396042) (end 145.9145 62.347542) (width 1.599) (layer "F.Cu") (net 1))
 (arc (start 105.9515 124.500999) (mid 105 123.5495) (end 104.0485 124.500999) (width 1.599) (layer "F.Cu") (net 1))
 (arc (start 138.3025 85.969999) (mid 139.254 86.9215) (end 140.205499 85.969999) (width 1.599) (layer "F.Cu") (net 1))
 (arc (start 119.2725 152.749) (mid 118.321 153.700499) (end 117.3695 152.749) (width 1.599) (layer "F.Cu") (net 1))
 (arc (start 109.055 111.6605) (mid 108.1035 112.612) (end 109.055 113.5635) (width 1.599) (layer "F.Cu") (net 1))
 (arc (start 57.251 119.2725) (mid 56.299499 118.321) (end 57.251 117.3695) (width 1.599) (layer "F.Cu") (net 1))
 (arc (start 65.988499 147.652457) (mid 65.036999 148.603957) (end 64.0855 147.652457) (width 1.599) (layer "F.Cu") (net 1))
 (arc (start 123.078499 152.749) (mid 122.127 153.700499) (end 121.175499 152.749) (width 1.599) (layer "F.Cu") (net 1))
 (arc (start 138.3025 152.749) (mid 137.351 153.700499) (end 136.3995 152.749) (width 1.599) (layer "F.Cu") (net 1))
 (arc (start 109.055 92.630499) (mid 108.1035 93.582) (end 109.055 94.533499) (width 1.599) (layer "F.Cu") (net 1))
 (arc (start 117.3695 62.85167) (mid 118.321 61.90017) (end 119.2725 62.85167) (width 1.599) (layer "F.Cu") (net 1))
 (arc (start 124.9815 124.029999) (mid 124.029999 123.078499) (end 123.078499 124.029999) (width 1.599) (layer "F.Cu") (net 1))
 (arc (start 73.6005 152.749) (mid 72.648999 153.700499) (end 71.697499 152.749) (width 1.599) (layer "F.Cu") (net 1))
 (arc (start 57.251 111.6605) (mid 56.299499 110.709) (end 57.251 109.7575) (width 1.599) (layer "F.Cu") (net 1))
 (arc (start 134.4965 85.969999) (mid 135.447999 86.9215) (end 136.3995 85.969999) (width 1.599) (layer "F.Cu") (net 1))
 (arc (start 104.0485 152.749) (mid 103.097 153.700499) (end 102.1455 152.749) (width 1.599) (layer "F.Cu") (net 1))
 (arc (start 64.0855 124.029999) (mid 63.133999 123.078499) (end 62.1825 124.029999) (width 1.599) (layer "F.Cu") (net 1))
 (arc (start 96.4365 152.749) (mid 95.485 153.700499) (end 94.533499 152.749) (width 1.599) (layer "F.Cu") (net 1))
 (arc (start 105.9515 59.154) (mid 106.902999 58.2025) (end 107.854499 59.154) (width 1.599) (layer "F.Cu") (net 1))
 (arc (start 109.055 107.854499) (mid 108.1035 108.806) (end 109.055 109.7575) (width 1.599) (layer "F.Cu") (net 1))
 (arc (start 109.055 88.8245) (mid 108.1035 89.776) (end 109.055 90.7275) (width 1.599) (layer "F.Cu") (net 1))
 (arc (start 58.3765 144.279078) (mid 57.425 145.230578) (end 56.473499 144.279078) (width 1.599) (layer "F.Cu") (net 1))
 (arc (start 103.345999 105.9515) (mid 105.364436 106.787563) (end 106.200499 108.805999) (width 1.599) (layer "F.Cu") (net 1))
 (arc (start 142.1085 85.969999) (mid 143.06 86.9215) (end 144.011499 85.969999) (width 1.599) (layer "F.Cu") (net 1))
 (arc (start 71.697499 124.029999) (mid 70.746 123.078499) (end 69.7945 124.029999) (width 1.599) (layer "F.Cu") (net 1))
 (arc (start 117.3695 124.029999) (mid 116.417999 123.078499) (end 115.4665 124.029999) (width 1.599) (layer "F.Cu") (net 1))
 (arc (start 100.999 121.175499) (mid 101.9505 120.224) (end 100.999 119.2725) (width 1.599) (layer "F.Cu") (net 1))
 (arc (start 69.7945 152.749) (mid 68.843 153.700499) (end 67.8915 152.749) (width 1.599) (layer "F.Cu") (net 1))
 (arc (start 152.749 90.7275) (mid 153.700499 91.679) (end 152.749 92.630499) (width 1.599) (layer "F.Cu") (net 1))
 (arc (start 60.2795 124.029999) (mid 59.327999 123.078499) (end 58.3765 124.029999) (width 1.599) (layer "F.Cu") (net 1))
 (arc (start 92.630499 152.749) (mid 91.679 153.700499) (end 90.7275 152.749) (width 1.599) (layer "F.Cu") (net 1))
 (arc (start 102.1455 124.029999) (mid 101.193999 123.078499) (end 100.2425 124.029999) (width 1.599) (layer "F.Cu") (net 1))
 (segment (start 102.1455 59.154) (end 102.1455 85.969999) (width 1.599) (layer "F.Cu") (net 2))
 (segment (start 58.3765 85.969999) (end 58.3765 65.720921) (width 1.599) (layer "F.Cu") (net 2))
 (segment (start 59.327999 88.8245) (end 100.999 88.8245) (width 1.599) (layer "F.Cu") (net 2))
 (segment (start 69.7945 85.969999) (end 69.7945 57.251) (width 1.599) (layer "F.Cu") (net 2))
 (segment (start 96.4365 85.969999) (end 96.4365 63.501) (width 1.599) (layer "F.Cu") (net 2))
 (segment (start 85.0185 85.969999) (end 85.0185 57.251) (width 1.599) (layer "F.Cu") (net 2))
 (segment (start 77.4065 85.969999) (end 77.4065 57.251) (width 1.599) (layer "F.Cu") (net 2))
 (segment (start 64.0855 62.347542) (end 64.0855 85.969999) (width 1.599) (layer "F.Cu") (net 2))
 (segment (start 90.7275 62.85167) (end 90.7275 85.969999) (width 1.599) (layer "F.Cu") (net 2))
 (segment (start 88.8245 85.969999) (end 88.8245 57.251) (width 1.599) (layer "F.Cu") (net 2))
 (segment (start 103.345999 98.3395) (end 57.251 98.3395) (width 1.599) (layer "F.Cu") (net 2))
 (segment (start 62.1825 85.969999) (end 62.1825 65.532537) (width 1.599) (layer "F.Cu") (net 2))
 (segment (start 57.251 96.4365) (end 103.345999 96.4365) (width 1.599) (layer "F.Cu") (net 2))
 (segment (start 57.251 100.2425) (end 103.345999 100.2425) (width 1.599) (layer "F.Cu") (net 2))
 (segment (start 57.251 92.630499) (end 101.209292 92.630499) (width 1.599) (layer "F.Cu") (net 2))
 (segment (start 94.533499 63.501) (end 94.533499 85.969999) (width 1.599) (layer "F.Cu") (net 2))
 (segment (start 83.1155 57.251) (end 83.1155 85.969999) (width 1.599) (layer "F.Cu") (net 2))
 (segment (start 60.2795 65.532537) (end 60.2795 85.969999) (width 1.599) (layer "F.Cu") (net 2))
 (segment (start 73.6005 85.969999) (end 73.6005 57.251) (width 1.599) (layer "F.Cu") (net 2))
 (segment (start 65.988499 85.969999) (end 65.988499 62.347542) (width 1.599) (layer "F.Cu") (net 2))
 (segment (start 81.212499 85.969999) (end 81.212499 57.251) (width 1.599) (layer "F.Cu") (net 2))
 (segment (start 103.345999 102.1455) (end 57.251 102.1455) (width 1.599) (layer "F.Cu") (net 2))
 (segment (start 98.3395 59.154) (end 98.3395 85.969999) (width 1.599) (layer "F.Cu") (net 2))
 (segment (start 67.8915 57.251) (end 67.8915 85.969999) (width 1.599) (layer "F.Cu") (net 2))
 (segment (start 56.473499 65.720921) (end 56.473499 85.969999) (width 1.599) (layer "F.Cu") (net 2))
 (segment (start 86.9215 57.251) (end 86.9215 85.969999) (width 1.599) (layer "F.Cu") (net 2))
 (segment (start 75.5035 57.251) (end 75.5035 85.969999) (width 1.599) (layer "F.Cu") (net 2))
 (segment (start 100.2425 85.969999) (end 100.2425 59.154) (width 1.599) (layer "F.Cu") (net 2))
 (segment (start 79.309499 57.251) (end 79.309499 85.969999) (width 1.599) (layer "F.Cu") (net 2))
 (segment (start 71.697499 57.251) (end 71.697499 85.969999) (width 1.599) (layer "F.Cu") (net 2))
 (segment (start 106.200499 90) (end 106.200499 101.194) (width 1.599) (layer "F.Cu") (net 2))
 (segment (start 95.29 56.299499) (end 99.291 56.299499) (width 1.599) (layer "F.Cu") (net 2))
 (segment (start 101.209292 94.533499) (end 57.251 94.533499) (width 1.599) (layer "F.Cu") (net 2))
 (segment (start 57.251 104.0485) (end 103.345999 104.0485) (width 1.599) (layer "F.Cu") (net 2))
 (segment (start 100.999 90.7275) (end 57.251 90.7275) (width 1.599) (layer "F.Cu") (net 2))
 (segment (start 92.630499 85.969999) (end 92.630499 62.85167) (width 1.599) (layer "F.Cu") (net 2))
 (arc (start 57.251 94.533499) (mid 56.299499 95.485) (end 57.251 96.4365) (width 1.599) (layer "F.Cu") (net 2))
 (arc (start 75.5035 85.969999) (mid 74.551999 86.9215) (end 73.6005 85.969999) (width 1.599) (layer "F.Cu") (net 2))
 (arc (start 65.988499 62.347542) (mid 65.036999 61.396042) (end 64.0855 62.347542) (width 1.599) (layer "F.Cu") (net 2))
 (arc (start 57.251 90.7275) (mid 56.299499 91.679) (end 57.251 92.630499) (width 1.599) (layer "F.Cu") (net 2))
 (arc (start 103.345999 100.2425) (mid 104.2975 101.193999) (end 103.345999 102.1455) (width 1.599) (layer "F.Cu") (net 2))
 (arc (start 71.697499 85.969999) (mid 70.746 86.9215) (end 69.7945 85.969999) (width 1.599) (layer "F.Cu") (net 2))
 (arc (start 83.1155 85.969999) (mid 82.164 86.9215) (end 81.212499 85.969999) (width 1.599) (layer "F.Cu") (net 2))
 (arc (start 81.212499 57.251) (mid 80.261 56.299499) (end 79.309499 57.251) (width 1.599) (layer "F.Cu") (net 2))
 (arc (start 79.309499 85.969999) (mid 78.358 86.9215) (end 77.4065 85.969999) (width 1.599) (layer "F.Cu") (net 2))
 (arc (start 103.345999 96.4365) (mid 104.2975 97.388) (end 103.345999 98.3395) (width 1.599) (layer "F.Cu") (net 2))
 (arc (start 100.999 88.8245) (mid 101.9505 89.776) (end 100.999 90.7275) (width 1.599) (layer "F.Cu") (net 2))
 (arc (start 57.251 102.1455) (mid 56.299499 103.097) (end 57.251 104.0485) (width 1.599) (layer "F.Cu") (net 2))
 (arc (start 86.9215 85.969999) (mid 85.969999 86.9215) (end 85.0185 85.969999) (width 1.599) (layer "F.Cu") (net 2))
 (arc (start 57.251 98.3395) (mid 56.299499 99.291) (end 57.251 100.2425) (width 1.599) (layer "F.Cu") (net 2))
 (arc (start 77.4065 57.251) (mid 76.455 56.299499) (end 75.5035 57.251) (width 1.599) (layer "F.Cu") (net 2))
 (arc (start 58.3765 65.720921) (mid 57.425 64.769421) (end 56.473499 65.720921) (width 1.599) (layer "F.Cu") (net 2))
 (arc (start 69.7945 57.251) (mid 68.843 56.299499) (end 67.8915 57.251) (width 1.599) (layer "F.Cu") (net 2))
 (arc (start 67.8915 85.969999) (mid 66.94 86.9215) (end 65.988499 85.969999) (width 1.599) (layer "F.Cu") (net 2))
 (arc (start 101.209292 92.630499) (mid 102.160793 93.582) (end 101.209292 94.533499) (width 1.599) (layer "F.Cu") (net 2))
 (arc (start 64.0855 85.969999) (mid 63.133999 86.9215) (end 62.1825 85.969999) (width 1.599) (layer "F.Cu") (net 2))
 (arc (start 92.630499 62.85167) (mid 91.679 61.900171) (end 90.7275 62.85167) (width 1.599) (layer "F.Cu") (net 2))
 (arc (start 106.200499 101.194) (mid 105.364436 103.212436) (end 103.345999 104.0485) (width 1.599) (layer "F.Cu") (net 2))
 (arc (start 62.1825 65.532537) (mid 61.230999 64.581037) (end 60.2795 65.532537) (width 1.599) (layer "F.Cu") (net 2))
 (arc (start 100.2425 59.154) (mid 99.291 58.2025) (end 98.3395 59.154) (width 1.599) (layer "F.Cu") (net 2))
 (arc (start 102.1455 85.969999) (mid 101.193999 86.9215) (end 100.2425 85.969999) (width 1.599) (layer "F.Cu") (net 2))
 (arc (start 96.4365 63.501) (mid 95.485 62.549499) (end 94.533499 63.501) (width 1.599) (layer "F.Cu") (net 2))
 (arc (start 88.8245 57.251) (mid 87.872999 56.299499) (end 86.9215 57.251) (width 1.599) (layer "F.Cu") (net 2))
 (arc (start 73.6005 57.251) (mid 72.648999 56.299499) (end 71.697499 57.251) (width 1.599) (layer "F.Cu") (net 2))
 (arc (start 85.0185 57.251) (mid 84.067 56.299499) (end 83.1155 57.251) (width 1.599) (layer "F.Cu") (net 2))
 (arc (start 59.327999 88.8245) (mid 57.309563 87.988436) (end 56.473499 85.969999) (width 1.599) (layer "F.Cu") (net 2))
 (arc (start 94.533499 85.969999) (mid 93.582 86.9215) (end 92.630499 85.969999) (width 1.599) (layer "F.Cu") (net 2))
 (arc (start 60.2795 85.969999) (mid 59.327999 86.9215) (end 58.3765 85.969999) (width 1.599) (layer "F.Cu") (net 2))
 (arc (start 90.7275 85.969999) (mid 89.776 86.9215) (end 88.8245 85.969999) (width 1.599) (layer "F.Cu") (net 2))
 (arc (start 99.291 56.299499) (mid 101.309436 57.135563) (end 102.1455 59.154) (width 1.599) (layer "F.Cu") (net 2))
 (arc (start 98.3395 85.969999) (mid 97.388 86.9215) (end 96.4365 85.969999) (width 1.599) (layer "F.Cu") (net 2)))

